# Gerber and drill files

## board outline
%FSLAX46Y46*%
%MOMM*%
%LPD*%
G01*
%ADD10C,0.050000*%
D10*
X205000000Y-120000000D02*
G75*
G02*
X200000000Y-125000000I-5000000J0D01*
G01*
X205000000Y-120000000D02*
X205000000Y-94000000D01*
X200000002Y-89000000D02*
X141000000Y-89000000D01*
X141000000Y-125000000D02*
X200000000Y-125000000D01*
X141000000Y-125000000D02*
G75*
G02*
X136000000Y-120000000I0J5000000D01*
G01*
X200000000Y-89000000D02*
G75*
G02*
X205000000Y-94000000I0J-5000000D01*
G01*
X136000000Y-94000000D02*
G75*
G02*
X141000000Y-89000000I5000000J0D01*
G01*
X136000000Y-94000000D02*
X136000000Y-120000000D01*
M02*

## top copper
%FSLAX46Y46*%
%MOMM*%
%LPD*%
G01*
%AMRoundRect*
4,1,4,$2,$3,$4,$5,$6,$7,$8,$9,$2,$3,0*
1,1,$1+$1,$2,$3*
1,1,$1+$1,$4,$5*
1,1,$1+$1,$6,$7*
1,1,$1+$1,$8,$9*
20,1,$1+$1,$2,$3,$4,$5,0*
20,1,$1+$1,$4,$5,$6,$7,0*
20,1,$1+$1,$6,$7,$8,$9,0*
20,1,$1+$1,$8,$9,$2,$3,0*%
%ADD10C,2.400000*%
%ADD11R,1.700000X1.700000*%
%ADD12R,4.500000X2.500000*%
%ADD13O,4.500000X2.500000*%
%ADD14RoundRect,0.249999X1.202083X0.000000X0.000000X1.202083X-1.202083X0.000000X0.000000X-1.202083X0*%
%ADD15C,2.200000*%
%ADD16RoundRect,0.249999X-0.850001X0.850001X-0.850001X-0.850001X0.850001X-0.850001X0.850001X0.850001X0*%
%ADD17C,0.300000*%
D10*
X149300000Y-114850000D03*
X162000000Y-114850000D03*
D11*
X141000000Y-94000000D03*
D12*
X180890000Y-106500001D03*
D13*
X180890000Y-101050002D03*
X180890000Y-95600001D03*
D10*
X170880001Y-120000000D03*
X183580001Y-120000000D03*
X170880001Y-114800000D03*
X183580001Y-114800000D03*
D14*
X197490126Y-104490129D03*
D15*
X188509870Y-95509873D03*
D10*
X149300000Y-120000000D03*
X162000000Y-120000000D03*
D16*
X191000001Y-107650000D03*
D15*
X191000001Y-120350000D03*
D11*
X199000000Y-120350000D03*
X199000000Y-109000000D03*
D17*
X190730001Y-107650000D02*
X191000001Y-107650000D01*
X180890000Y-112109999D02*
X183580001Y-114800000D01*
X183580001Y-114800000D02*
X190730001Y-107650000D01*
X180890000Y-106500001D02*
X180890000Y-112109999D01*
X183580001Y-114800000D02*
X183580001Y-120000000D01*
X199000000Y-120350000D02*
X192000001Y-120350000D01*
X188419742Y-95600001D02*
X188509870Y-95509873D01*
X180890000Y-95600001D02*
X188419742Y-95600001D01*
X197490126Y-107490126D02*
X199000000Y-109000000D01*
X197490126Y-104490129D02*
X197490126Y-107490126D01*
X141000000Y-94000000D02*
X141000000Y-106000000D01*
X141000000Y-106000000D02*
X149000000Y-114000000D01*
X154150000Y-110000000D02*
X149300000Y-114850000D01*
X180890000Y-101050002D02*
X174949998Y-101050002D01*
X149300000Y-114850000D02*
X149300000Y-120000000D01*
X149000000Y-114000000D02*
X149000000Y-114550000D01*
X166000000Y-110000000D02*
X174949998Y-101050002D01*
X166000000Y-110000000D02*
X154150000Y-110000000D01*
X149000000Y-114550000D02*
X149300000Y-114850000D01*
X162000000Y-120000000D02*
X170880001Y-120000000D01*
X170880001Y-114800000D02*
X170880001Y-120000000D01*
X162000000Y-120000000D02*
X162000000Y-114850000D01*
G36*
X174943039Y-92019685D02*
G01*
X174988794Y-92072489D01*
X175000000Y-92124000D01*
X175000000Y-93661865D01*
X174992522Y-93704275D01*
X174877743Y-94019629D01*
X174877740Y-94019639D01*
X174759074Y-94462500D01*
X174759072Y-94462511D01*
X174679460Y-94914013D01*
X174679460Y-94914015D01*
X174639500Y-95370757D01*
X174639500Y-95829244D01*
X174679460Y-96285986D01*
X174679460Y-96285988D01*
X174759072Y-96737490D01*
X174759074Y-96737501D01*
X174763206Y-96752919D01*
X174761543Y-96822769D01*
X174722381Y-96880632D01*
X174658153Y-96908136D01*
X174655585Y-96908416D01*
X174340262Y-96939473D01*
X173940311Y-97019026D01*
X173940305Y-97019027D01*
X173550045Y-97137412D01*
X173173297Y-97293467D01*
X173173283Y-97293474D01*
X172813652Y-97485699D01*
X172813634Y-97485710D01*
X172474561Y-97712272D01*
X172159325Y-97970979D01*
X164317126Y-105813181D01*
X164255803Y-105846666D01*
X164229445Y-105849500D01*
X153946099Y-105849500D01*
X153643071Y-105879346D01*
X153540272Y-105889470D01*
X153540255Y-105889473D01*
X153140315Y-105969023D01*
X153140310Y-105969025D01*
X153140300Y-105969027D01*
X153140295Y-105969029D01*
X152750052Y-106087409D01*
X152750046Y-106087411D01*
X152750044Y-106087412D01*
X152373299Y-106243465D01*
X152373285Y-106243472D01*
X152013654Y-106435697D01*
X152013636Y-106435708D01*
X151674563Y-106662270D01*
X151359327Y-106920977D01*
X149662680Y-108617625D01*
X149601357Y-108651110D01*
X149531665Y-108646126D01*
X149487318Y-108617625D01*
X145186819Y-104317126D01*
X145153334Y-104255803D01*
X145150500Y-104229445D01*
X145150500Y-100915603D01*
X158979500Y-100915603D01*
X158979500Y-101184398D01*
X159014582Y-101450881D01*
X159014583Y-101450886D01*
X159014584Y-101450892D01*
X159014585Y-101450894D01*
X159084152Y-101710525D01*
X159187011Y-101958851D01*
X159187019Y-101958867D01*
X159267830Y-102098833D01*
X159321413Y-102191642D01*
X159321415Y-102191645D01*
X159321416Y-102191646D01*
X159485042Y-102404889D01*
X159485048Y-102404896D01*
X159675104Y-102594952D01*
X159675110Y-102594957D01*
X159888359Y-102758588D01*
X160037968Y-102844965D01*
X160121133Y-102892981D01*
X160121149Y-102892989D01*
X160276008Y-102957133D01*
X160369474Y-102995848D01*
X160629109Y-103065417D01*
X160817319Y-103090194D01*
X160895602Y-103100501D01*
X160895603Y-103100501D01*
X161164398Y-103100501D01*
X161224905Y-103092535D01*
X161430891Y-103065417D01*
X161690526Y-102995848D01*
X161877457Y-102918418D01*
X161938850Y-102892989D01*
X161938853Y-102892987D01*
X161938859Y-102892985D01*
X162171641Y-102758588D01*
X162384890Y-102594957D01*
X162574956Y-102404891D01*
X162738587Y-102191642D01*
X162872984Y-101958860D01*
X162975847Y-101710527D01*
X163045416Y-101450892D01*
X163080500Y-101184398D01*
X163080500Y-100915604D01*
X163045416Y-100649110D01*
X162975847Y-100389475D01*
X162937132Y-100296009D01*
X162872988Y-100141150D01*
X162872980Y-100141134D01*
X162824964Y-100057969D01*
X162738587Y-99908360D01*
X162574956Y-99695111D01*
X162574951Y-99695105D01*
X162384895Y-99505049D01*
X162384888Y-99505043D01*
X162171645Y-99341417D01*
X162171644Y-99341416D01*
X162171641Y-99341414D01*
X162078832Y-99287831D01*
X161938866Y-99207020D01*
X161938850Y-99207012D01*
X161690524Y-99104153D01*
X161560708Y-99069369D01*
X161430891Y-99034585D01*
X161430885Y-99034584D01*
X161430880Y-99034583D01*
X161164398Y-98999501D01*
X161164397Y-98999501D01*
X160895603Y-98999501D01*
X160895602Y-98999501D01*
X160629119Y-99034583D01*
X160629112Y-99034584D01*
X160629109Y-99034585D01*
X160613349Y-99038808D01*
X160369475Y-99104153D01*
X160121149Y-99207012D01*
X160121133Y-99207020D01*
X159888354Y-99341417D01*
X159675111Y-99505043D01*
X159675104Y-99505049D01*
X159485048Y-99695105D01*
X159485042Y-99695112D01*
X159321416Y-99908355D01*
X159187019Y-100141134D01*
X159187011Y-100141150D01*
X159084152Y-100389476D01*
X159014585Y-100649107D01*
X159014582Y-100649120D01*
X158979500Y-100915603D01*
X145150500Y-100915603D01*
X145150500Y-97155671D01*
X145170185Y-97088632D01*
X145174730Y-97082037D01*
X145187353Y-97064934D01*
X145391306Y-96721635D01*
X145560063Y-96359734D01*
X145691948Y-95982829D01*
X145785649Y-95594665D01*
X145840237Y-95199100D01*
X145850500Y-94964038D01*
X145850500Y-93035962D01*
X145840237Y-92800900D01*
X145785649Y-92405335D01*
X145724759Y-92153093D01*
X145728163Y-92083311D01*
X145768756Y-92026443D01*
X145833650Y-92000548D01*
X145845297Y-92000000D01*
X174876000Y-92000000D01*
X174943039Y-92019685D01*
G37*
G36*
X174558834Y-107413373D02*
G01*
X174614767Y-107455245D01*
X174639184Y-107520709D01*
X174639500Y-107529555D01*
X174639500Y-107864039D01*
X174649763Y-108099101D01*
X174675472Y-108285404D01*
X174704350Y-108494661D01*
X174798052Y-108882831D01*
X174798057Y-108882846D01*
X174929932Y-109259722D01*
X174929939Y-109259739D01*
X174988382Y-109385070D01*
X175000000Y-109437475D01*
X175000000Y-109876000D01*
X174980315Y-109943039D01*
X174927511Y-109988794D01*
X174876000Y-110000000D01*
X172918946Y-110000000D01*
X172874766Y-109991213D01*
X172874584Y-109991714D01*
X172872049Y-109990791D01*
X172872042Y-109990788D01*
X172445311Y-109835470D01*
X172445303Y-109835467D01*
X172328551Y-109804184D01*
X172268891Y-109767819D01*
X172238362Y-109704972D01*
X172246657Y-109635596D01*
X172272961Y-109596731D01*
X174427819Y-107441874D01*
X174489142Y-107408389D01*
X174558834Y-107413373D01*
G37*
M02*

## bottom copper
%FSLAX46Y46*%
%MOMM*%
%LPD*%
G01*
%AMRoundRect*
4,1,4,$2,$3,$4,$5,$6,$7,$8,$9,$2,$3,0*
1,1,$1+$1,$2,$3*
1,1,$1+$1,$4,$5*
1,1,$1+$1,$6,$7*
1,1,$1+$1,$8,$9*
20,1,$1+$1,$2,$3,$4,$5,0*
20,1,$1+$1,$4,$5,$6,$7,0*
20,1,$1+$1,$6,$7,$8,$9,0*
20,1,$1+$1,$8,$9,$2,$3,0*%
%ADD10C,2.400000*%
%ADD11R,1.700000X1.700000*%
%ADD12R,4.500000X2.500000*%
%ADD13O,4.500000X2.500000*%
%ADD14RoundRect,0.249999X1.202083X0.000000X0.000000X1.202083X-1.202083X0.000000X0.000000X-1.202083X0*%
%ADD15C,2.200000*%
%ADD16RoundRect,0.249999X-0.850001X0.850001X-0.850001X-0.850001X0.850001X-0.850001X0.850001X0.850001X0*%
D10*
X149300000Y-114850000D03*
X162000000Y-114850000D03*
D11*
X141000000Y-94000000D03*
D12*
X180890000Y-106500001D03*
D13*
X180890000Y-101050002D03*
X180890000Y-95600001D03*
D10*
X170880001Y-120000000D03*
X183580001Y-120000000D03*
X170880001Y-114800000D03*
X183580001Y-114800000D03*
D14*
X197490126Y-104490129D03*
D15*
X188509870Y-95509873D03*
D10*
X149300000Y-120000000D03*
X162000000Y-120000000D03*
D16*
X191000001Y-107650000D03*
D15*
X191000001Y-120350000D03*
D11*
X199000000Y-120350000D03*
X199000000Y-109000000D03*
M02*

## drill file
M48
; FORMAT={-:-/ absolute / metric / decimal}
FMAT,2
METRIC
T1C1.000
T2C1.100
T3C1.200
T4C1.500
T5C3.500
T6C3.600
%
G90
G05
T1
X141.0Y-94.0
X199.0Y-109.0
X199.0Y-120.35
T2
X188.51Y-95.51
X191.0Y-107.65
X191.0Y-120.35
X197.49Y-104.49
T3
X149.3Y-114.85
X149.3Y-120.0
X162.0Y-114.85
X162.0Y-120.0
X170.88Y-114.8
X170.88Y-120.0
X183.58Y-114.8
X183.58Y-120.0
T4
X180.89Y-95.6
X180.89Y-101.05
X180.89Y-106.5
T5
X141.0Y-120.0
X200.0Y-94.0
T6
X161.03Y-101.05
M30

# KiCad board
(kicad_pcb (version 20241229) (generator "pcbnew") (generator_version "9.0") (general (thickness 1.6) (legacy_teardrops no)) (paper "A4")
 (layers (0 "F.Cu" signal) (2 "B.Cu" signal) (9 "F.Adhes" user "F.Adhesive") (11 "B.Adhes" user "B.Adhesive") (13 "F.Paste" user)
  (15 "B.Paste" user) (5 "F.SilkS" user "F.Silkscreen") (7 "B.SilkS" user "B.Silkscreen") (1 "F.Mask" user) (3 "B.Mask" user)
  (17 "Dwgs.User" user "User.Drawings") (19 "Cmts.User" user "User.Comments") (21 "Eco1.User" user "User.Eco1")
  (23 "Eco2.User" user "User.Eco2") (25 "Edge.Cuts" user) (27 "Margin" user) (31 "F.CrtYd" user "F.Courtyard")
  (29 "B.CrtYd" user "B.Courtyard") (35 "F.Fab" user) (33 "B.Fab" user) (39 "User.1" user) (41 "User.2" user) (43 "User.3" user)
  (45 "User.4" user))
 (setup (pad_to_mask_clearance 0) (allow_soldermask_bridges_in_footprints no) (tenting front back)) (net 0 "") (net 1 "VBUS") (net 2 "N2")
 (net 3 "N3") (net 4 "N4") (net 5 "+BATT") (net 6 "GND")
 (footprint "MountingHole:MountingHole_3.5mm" (layer "F.Cu") (at 141 120)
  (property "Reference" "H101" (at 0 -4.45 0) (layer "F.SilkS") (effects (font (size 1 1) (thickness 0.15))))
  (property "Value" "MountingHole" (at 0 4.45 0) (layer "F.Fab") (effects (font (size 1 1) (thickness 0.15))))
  (pad "" np_thru_hole circle (at 0 0) (size 3.5 3.5) (drill 3.5) (layers "*.Cu" "*.Mask")))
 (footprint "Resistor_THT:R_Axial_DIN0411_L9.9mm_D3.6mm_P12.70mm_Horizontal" (layer "F.Cu") (at 149.3 114.85)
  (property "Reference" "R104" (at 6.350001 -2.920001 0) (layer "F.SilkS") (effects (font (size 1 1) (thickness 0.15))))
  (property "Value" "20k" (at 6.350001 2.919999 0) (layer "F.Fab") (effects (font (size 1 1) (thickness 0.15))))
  (pad "1" thru_hole circle (at 0 0) (size 2.4 2.4) (drill 1.2) (layers "*.Cu" "*.Mask") (remove_unused_layers no) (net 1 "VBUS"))
  (pad "2" thru_hole circle (at 12.7 0) (size 2.4 2.4) (drill 1.2) (layers "*.Cu" "*.Mask") (remove_unused_layers no) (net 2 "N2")))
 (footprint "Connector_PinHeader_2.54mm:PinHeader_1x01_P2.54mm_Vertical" (layer "F.Cu") (at 141 94)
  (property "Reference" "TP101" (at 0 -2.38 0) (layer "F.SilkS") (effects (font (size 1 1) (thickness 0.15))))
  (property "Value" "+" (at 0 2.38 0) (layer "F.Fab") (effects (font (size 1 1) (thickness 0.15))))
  (pad "1" thru_hole rect (at 0 0) (size 1.7 1.7) (drill 1) (layers "*.Cu" "*.Mask") (remove_unused_layers no) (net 1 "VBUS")))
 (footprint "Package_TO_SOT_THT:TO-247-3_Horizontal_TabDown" (layer "F.Cu") (at 180.89 106.500001 90)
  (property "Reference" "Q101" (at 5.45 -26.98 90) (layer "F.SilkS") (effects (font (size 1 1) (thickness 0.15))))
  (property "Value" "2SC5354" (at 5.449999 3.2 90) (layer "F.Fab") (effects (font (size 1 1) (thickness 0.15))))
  (pad "" np_thru_hole circle (at 5.45 -19.86 90) (size 3.6 3.6) (drill 3.6) (layers "*.Cu" "*.Mask"))
  (pad "1" thru_hole rect (at 0 0 90) (size 2.5 4.5) (drill 1.5) (layers "*.Cu" "*.Mask") (remove_unused_layers no) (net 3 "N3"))
  (pad "2" thru_hole oval (at 5.449999 0 90) (size 2.5 4.5) (drill 1.5) (layers "*.Cu" "*.Mask") (remove_unused_layers no) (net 1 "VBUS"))
  (pad "3" thru_hole oval (at 10.9 0 90) (size 2.5 4.5) (drill 1.5) (layers "*.Cu" "*.Mask") (remove_unused_layers no) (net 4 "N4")))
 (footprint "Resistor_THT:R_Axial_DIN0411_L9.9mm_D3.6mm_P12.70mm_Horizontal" (layer "F.Cu") (at 170.880001 120)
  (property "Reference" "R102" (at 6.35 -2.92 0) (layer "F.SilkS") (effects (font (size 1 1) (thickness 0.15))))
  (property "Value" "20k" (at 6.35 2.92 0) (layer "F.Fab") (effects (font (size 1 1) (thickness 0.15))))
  (pad "1" thru_hole circle (at 0 0) (size 2.4 2.4) (drill 1.2) (layers "*.Cu" "*.Mask") (remove_unused_layers no) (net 2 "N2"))
  (pad "2" thru_hole circle (at 12.7 0) (size 2.4 2.4) (drill 1.2) (layers "*.Cu" "*.Mask") (remove_unused_layers no) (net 3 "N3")))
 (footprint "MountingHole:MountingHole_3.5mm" (layer "F.Cu") (at 200 94)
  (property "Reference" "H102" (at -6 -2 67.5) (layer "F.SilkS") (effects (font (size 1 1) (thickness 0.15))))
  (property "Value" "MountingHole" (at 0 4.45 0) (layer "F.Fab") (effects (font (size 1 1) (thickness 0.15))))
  (pad "" np_thru_hole circle (at 0 0) (size 3.5 3.5) (drill 3.5) (layers "*.Cu" "*.Mask")))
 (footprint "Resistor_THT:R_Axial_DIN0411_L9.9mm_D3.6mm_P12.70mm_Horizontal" (layer "F.Cu") (at 170.880001 114.8)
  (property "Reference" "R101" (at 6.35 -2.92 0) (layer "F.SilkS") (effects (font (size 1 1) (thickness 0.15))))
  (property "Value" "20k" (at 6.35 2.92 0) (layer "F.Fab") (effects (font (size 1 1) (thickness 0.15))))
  (pad "1" thru_hole circle (at 0 0) (size 2.4 2.4) (drill 1.2) (layers "*.Cu" "*.Mask") (remove_unused_layers no) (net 2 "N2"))
  (pad "2" thru_hole circle (at 12.7 0) (size 2.4 2.4) (drill 1.2) (layers "*.Cu" "*.Mask") (remove_unused_layers no) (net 3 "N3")))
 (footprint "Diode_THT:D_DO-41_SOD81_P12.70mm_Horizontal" (layer "F.Cu") (at 197.490126 104.490129 135)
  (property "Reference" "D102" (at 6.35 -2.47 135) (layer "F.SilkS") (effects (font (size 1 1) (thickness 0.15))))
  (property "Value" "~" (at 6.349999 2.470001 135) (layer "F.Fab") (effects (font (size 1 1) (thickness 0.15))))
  (pad "1" thru_hole roundrect (at 0 0 135) (size 2.2 2.2) (drill 1.1) (layers "*.Cu" "*.Mask") (remove_unused_layers no)
   (roundrect_rratio 0.113636) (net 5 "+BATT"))
  (pad "2" thru_hole circle (at 12.7 0 135) (size 2.2 2.2) (drill 1.1) (layers "*.Cu" "*.Mask") (remove_unused_layers no) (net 4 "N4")))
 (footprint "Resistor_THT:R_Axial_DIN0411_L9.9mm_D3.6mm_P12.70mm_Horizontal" (layer "F.Cu") (at 149.3 120)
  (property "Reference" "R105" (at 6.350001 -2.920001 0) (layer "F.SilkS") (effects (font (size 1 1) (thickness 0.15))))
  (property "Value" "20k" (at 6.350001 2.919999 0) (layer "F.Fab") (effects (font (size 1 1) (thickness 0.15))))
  (pad "1" thru_hole circle (at 0 0) (size 2.4 2.4) (drill 1.2) (layers "*.Cu" "*.Mask") (remove_unused_layers no) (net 1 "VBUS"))
  (pad "2" thru_hole circle (at 12.7 0) (size 2.4 2.4) (drill 1.2) (layers "*.Cu" "*.Mask") (remove_unused_layers no) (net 2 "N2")))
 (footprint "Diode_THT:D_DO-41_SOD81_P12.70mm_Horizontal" (layer "F.Cu") (at 191.000001 107.65 -90)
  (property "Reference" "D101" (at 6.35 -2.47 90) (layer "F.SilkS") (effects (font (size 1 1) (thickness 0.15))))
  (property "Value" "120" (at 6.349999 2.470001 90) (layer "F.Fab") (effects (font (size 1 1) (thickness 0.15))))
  (pad "1" thru_hole roundrect (at 0 0 270) (size 2.2 2.2) (drill 1.1) (layers "*.Cu" "*.Mask") (remove_unused_layers no)
   (roundrect_rratio 0.113636) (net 3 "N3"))
  (pad "2" thru_hole circle (at 12.7 0 270) (size 2.2 2.2) (drill 1.1) (layers "*.Cu" "*.Mask") (remove_unused_layers no) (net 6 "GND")))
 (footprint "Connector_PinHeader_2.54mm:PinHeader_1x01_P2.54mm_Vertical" (layer "F.Cu") (at 199 120.35)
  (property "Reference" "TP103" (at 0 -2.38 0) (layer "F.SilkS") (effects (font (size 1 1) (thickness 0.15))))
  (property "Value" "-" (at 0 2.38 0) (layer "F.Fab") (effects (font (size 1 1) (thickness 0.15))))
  (pad "1" thru_hole rect (at 0 0) (size 1.7 1.7) (drill 1) (layers "*.Cu" "*.Mask") (remove_unused_layers no) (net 6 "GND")))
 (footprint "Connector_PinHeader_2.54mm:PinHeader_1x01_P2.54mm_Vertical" (layer "F.Cu") (at 199 109)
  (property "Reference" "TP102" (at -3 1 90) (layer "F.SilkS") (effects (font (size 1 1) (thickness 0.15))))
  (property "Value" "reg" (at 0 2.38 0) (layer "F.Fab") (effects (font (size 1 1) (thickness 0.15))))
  (pad "1" thru_hole rect (at 0 0) (size 1.7 1.7) (drill 1) (layers "*.Cu" "*.Mask") (remove_unused_layers no) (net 5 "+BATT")))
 (gr_arc (start 205 120) (mid 203.535534 123.535534) (end 200 125) (stroke (width 0.05) (type default)) (layer "Edge.Cuts"))
 (gr_line (start 205 120) (end 205 94) (stroke (width 0.05) (type default)) (layer "Edge.Cuts"))
 (gr_line (start 200.000002 89) (end 141 89) (stroke (width 0.05) (type default)) (layer "Edge.Cuts"))
 (gr_line (start 141 125) (end 200 125) (stroke (width 0.05) (type default)) (layer "Edge.Cuts"))
 (gr_arc (start 141 125) (mid 137.464466 123.535534) (end 136 120) (stroke (width 0.05) (type default)) (layer "Edge.Cuts"))
 (gr_arc (start 200 89) (mid 203.535534 90.464466) (end 205 94) (stroke (width 0.05) (type default)) (layer "Edge.Cuts"))
 (gr_arc (start 136 94) (mid 137.464466 90.464466) (end 141 89) (stroke (width 0.05) (type default)) (layer "Edge.Cuts"))
 (gr_line (start 136 94) (end 136 120) (stroke (width 0.05) (type default)) (layer "Edge.Cuts"))
 (segment (start 190.730001 107.65) (end 191.000001 107.65) (width 0.3) (layer "F.Cu") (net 3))
 (segment (start 180.89 112.109999) (end 183.580001 114.8) (width 0.3) (layer "F.Cu") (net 3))
 (segment (start 183.580001 114.8) (end 190.730001 107.65) (width 0.3) (layer "F.Cu") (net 3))
 (segment (start 180.89 106.500001) (end 180.89 112.109999) (width 0.3) (layer "F.Cu") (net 3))
 (segment (start 183.580001 114.8) (end 183.580001 120) (width 0.3) (layer "F.Cu") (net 3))
 (segment (start 199 120.35) (end 192.000001 120.35) (width 0.3) (layer "F.Cu") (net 6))
 (segment (start 188.419742 95.600001) (end 188.50987 95.509873) (width 0.3) (layer "F.Cu") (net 4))
 (segment (start 180.89 95.600001) (end 188.419742 95.600001) (width 0.3) (layer "F.Cu") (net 4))
 (segment (start 197.490126 107.490126) (end 199 109) (width 0.3) (layer "F.Cu") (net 5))
 (segment (start 197.490126 104.490129) (end 197.490126 107.490126) (width 0.3) (layer "F.Cu") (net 5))
 (segment (start 141 94) (end 141 106) (width 0.3) (layer "F.Cu") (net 1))
 (segment (start 141 106) (end 149 114) (width 0.3) (layer "F.Cu") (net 1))
 (segment (start 154.15 110) (end 149.3 114.85) (width 0.3) (layer "F.Cu") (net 1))
 (segment (start 180.89 101.050002) (end 174.949998 101.050002) (width 0.3) (layer "F.Cu") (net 1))
 (segment (start 149.3 114.85) (end 149.3 120) (width 0.3) (layer "F.Cu") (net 1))
 (segment (start 149 114) (end 149 114.55) (width 0.3) (layer "F.Cu") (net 1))
 (segment (start 166 110) (end 174.949998 101.050002) (width 0.3) (layer "F.Cu") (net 1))
 (segment (start 166 110) (end 154.15 110) (width 0.3) (layer "F.Cu") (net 1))
 (segment (start 149 114.55) (end 149.3 114.85) (width 0.3) (layer "F.Cu") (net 1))
 (segment (start 162 120) (end 170.880001 120) (width 0.3) (layer "F.Cu") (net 2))
 (segment (start 170.880001 114.8) (end 170.880001 120) (width 0.3) (layer "F.Cu") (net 2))
 (segment (start 162 120) (end 162 114.85) (width 0.3) (layer "F.Cu") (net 2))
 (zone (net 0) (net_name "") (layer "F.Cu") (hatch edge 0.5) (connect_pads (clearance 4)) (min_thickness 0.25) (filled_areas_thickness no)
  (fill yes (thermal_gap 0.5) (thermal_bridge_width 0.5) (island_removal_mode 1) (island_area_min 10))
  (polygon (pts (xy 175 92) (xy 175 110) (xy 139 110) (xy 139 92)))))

